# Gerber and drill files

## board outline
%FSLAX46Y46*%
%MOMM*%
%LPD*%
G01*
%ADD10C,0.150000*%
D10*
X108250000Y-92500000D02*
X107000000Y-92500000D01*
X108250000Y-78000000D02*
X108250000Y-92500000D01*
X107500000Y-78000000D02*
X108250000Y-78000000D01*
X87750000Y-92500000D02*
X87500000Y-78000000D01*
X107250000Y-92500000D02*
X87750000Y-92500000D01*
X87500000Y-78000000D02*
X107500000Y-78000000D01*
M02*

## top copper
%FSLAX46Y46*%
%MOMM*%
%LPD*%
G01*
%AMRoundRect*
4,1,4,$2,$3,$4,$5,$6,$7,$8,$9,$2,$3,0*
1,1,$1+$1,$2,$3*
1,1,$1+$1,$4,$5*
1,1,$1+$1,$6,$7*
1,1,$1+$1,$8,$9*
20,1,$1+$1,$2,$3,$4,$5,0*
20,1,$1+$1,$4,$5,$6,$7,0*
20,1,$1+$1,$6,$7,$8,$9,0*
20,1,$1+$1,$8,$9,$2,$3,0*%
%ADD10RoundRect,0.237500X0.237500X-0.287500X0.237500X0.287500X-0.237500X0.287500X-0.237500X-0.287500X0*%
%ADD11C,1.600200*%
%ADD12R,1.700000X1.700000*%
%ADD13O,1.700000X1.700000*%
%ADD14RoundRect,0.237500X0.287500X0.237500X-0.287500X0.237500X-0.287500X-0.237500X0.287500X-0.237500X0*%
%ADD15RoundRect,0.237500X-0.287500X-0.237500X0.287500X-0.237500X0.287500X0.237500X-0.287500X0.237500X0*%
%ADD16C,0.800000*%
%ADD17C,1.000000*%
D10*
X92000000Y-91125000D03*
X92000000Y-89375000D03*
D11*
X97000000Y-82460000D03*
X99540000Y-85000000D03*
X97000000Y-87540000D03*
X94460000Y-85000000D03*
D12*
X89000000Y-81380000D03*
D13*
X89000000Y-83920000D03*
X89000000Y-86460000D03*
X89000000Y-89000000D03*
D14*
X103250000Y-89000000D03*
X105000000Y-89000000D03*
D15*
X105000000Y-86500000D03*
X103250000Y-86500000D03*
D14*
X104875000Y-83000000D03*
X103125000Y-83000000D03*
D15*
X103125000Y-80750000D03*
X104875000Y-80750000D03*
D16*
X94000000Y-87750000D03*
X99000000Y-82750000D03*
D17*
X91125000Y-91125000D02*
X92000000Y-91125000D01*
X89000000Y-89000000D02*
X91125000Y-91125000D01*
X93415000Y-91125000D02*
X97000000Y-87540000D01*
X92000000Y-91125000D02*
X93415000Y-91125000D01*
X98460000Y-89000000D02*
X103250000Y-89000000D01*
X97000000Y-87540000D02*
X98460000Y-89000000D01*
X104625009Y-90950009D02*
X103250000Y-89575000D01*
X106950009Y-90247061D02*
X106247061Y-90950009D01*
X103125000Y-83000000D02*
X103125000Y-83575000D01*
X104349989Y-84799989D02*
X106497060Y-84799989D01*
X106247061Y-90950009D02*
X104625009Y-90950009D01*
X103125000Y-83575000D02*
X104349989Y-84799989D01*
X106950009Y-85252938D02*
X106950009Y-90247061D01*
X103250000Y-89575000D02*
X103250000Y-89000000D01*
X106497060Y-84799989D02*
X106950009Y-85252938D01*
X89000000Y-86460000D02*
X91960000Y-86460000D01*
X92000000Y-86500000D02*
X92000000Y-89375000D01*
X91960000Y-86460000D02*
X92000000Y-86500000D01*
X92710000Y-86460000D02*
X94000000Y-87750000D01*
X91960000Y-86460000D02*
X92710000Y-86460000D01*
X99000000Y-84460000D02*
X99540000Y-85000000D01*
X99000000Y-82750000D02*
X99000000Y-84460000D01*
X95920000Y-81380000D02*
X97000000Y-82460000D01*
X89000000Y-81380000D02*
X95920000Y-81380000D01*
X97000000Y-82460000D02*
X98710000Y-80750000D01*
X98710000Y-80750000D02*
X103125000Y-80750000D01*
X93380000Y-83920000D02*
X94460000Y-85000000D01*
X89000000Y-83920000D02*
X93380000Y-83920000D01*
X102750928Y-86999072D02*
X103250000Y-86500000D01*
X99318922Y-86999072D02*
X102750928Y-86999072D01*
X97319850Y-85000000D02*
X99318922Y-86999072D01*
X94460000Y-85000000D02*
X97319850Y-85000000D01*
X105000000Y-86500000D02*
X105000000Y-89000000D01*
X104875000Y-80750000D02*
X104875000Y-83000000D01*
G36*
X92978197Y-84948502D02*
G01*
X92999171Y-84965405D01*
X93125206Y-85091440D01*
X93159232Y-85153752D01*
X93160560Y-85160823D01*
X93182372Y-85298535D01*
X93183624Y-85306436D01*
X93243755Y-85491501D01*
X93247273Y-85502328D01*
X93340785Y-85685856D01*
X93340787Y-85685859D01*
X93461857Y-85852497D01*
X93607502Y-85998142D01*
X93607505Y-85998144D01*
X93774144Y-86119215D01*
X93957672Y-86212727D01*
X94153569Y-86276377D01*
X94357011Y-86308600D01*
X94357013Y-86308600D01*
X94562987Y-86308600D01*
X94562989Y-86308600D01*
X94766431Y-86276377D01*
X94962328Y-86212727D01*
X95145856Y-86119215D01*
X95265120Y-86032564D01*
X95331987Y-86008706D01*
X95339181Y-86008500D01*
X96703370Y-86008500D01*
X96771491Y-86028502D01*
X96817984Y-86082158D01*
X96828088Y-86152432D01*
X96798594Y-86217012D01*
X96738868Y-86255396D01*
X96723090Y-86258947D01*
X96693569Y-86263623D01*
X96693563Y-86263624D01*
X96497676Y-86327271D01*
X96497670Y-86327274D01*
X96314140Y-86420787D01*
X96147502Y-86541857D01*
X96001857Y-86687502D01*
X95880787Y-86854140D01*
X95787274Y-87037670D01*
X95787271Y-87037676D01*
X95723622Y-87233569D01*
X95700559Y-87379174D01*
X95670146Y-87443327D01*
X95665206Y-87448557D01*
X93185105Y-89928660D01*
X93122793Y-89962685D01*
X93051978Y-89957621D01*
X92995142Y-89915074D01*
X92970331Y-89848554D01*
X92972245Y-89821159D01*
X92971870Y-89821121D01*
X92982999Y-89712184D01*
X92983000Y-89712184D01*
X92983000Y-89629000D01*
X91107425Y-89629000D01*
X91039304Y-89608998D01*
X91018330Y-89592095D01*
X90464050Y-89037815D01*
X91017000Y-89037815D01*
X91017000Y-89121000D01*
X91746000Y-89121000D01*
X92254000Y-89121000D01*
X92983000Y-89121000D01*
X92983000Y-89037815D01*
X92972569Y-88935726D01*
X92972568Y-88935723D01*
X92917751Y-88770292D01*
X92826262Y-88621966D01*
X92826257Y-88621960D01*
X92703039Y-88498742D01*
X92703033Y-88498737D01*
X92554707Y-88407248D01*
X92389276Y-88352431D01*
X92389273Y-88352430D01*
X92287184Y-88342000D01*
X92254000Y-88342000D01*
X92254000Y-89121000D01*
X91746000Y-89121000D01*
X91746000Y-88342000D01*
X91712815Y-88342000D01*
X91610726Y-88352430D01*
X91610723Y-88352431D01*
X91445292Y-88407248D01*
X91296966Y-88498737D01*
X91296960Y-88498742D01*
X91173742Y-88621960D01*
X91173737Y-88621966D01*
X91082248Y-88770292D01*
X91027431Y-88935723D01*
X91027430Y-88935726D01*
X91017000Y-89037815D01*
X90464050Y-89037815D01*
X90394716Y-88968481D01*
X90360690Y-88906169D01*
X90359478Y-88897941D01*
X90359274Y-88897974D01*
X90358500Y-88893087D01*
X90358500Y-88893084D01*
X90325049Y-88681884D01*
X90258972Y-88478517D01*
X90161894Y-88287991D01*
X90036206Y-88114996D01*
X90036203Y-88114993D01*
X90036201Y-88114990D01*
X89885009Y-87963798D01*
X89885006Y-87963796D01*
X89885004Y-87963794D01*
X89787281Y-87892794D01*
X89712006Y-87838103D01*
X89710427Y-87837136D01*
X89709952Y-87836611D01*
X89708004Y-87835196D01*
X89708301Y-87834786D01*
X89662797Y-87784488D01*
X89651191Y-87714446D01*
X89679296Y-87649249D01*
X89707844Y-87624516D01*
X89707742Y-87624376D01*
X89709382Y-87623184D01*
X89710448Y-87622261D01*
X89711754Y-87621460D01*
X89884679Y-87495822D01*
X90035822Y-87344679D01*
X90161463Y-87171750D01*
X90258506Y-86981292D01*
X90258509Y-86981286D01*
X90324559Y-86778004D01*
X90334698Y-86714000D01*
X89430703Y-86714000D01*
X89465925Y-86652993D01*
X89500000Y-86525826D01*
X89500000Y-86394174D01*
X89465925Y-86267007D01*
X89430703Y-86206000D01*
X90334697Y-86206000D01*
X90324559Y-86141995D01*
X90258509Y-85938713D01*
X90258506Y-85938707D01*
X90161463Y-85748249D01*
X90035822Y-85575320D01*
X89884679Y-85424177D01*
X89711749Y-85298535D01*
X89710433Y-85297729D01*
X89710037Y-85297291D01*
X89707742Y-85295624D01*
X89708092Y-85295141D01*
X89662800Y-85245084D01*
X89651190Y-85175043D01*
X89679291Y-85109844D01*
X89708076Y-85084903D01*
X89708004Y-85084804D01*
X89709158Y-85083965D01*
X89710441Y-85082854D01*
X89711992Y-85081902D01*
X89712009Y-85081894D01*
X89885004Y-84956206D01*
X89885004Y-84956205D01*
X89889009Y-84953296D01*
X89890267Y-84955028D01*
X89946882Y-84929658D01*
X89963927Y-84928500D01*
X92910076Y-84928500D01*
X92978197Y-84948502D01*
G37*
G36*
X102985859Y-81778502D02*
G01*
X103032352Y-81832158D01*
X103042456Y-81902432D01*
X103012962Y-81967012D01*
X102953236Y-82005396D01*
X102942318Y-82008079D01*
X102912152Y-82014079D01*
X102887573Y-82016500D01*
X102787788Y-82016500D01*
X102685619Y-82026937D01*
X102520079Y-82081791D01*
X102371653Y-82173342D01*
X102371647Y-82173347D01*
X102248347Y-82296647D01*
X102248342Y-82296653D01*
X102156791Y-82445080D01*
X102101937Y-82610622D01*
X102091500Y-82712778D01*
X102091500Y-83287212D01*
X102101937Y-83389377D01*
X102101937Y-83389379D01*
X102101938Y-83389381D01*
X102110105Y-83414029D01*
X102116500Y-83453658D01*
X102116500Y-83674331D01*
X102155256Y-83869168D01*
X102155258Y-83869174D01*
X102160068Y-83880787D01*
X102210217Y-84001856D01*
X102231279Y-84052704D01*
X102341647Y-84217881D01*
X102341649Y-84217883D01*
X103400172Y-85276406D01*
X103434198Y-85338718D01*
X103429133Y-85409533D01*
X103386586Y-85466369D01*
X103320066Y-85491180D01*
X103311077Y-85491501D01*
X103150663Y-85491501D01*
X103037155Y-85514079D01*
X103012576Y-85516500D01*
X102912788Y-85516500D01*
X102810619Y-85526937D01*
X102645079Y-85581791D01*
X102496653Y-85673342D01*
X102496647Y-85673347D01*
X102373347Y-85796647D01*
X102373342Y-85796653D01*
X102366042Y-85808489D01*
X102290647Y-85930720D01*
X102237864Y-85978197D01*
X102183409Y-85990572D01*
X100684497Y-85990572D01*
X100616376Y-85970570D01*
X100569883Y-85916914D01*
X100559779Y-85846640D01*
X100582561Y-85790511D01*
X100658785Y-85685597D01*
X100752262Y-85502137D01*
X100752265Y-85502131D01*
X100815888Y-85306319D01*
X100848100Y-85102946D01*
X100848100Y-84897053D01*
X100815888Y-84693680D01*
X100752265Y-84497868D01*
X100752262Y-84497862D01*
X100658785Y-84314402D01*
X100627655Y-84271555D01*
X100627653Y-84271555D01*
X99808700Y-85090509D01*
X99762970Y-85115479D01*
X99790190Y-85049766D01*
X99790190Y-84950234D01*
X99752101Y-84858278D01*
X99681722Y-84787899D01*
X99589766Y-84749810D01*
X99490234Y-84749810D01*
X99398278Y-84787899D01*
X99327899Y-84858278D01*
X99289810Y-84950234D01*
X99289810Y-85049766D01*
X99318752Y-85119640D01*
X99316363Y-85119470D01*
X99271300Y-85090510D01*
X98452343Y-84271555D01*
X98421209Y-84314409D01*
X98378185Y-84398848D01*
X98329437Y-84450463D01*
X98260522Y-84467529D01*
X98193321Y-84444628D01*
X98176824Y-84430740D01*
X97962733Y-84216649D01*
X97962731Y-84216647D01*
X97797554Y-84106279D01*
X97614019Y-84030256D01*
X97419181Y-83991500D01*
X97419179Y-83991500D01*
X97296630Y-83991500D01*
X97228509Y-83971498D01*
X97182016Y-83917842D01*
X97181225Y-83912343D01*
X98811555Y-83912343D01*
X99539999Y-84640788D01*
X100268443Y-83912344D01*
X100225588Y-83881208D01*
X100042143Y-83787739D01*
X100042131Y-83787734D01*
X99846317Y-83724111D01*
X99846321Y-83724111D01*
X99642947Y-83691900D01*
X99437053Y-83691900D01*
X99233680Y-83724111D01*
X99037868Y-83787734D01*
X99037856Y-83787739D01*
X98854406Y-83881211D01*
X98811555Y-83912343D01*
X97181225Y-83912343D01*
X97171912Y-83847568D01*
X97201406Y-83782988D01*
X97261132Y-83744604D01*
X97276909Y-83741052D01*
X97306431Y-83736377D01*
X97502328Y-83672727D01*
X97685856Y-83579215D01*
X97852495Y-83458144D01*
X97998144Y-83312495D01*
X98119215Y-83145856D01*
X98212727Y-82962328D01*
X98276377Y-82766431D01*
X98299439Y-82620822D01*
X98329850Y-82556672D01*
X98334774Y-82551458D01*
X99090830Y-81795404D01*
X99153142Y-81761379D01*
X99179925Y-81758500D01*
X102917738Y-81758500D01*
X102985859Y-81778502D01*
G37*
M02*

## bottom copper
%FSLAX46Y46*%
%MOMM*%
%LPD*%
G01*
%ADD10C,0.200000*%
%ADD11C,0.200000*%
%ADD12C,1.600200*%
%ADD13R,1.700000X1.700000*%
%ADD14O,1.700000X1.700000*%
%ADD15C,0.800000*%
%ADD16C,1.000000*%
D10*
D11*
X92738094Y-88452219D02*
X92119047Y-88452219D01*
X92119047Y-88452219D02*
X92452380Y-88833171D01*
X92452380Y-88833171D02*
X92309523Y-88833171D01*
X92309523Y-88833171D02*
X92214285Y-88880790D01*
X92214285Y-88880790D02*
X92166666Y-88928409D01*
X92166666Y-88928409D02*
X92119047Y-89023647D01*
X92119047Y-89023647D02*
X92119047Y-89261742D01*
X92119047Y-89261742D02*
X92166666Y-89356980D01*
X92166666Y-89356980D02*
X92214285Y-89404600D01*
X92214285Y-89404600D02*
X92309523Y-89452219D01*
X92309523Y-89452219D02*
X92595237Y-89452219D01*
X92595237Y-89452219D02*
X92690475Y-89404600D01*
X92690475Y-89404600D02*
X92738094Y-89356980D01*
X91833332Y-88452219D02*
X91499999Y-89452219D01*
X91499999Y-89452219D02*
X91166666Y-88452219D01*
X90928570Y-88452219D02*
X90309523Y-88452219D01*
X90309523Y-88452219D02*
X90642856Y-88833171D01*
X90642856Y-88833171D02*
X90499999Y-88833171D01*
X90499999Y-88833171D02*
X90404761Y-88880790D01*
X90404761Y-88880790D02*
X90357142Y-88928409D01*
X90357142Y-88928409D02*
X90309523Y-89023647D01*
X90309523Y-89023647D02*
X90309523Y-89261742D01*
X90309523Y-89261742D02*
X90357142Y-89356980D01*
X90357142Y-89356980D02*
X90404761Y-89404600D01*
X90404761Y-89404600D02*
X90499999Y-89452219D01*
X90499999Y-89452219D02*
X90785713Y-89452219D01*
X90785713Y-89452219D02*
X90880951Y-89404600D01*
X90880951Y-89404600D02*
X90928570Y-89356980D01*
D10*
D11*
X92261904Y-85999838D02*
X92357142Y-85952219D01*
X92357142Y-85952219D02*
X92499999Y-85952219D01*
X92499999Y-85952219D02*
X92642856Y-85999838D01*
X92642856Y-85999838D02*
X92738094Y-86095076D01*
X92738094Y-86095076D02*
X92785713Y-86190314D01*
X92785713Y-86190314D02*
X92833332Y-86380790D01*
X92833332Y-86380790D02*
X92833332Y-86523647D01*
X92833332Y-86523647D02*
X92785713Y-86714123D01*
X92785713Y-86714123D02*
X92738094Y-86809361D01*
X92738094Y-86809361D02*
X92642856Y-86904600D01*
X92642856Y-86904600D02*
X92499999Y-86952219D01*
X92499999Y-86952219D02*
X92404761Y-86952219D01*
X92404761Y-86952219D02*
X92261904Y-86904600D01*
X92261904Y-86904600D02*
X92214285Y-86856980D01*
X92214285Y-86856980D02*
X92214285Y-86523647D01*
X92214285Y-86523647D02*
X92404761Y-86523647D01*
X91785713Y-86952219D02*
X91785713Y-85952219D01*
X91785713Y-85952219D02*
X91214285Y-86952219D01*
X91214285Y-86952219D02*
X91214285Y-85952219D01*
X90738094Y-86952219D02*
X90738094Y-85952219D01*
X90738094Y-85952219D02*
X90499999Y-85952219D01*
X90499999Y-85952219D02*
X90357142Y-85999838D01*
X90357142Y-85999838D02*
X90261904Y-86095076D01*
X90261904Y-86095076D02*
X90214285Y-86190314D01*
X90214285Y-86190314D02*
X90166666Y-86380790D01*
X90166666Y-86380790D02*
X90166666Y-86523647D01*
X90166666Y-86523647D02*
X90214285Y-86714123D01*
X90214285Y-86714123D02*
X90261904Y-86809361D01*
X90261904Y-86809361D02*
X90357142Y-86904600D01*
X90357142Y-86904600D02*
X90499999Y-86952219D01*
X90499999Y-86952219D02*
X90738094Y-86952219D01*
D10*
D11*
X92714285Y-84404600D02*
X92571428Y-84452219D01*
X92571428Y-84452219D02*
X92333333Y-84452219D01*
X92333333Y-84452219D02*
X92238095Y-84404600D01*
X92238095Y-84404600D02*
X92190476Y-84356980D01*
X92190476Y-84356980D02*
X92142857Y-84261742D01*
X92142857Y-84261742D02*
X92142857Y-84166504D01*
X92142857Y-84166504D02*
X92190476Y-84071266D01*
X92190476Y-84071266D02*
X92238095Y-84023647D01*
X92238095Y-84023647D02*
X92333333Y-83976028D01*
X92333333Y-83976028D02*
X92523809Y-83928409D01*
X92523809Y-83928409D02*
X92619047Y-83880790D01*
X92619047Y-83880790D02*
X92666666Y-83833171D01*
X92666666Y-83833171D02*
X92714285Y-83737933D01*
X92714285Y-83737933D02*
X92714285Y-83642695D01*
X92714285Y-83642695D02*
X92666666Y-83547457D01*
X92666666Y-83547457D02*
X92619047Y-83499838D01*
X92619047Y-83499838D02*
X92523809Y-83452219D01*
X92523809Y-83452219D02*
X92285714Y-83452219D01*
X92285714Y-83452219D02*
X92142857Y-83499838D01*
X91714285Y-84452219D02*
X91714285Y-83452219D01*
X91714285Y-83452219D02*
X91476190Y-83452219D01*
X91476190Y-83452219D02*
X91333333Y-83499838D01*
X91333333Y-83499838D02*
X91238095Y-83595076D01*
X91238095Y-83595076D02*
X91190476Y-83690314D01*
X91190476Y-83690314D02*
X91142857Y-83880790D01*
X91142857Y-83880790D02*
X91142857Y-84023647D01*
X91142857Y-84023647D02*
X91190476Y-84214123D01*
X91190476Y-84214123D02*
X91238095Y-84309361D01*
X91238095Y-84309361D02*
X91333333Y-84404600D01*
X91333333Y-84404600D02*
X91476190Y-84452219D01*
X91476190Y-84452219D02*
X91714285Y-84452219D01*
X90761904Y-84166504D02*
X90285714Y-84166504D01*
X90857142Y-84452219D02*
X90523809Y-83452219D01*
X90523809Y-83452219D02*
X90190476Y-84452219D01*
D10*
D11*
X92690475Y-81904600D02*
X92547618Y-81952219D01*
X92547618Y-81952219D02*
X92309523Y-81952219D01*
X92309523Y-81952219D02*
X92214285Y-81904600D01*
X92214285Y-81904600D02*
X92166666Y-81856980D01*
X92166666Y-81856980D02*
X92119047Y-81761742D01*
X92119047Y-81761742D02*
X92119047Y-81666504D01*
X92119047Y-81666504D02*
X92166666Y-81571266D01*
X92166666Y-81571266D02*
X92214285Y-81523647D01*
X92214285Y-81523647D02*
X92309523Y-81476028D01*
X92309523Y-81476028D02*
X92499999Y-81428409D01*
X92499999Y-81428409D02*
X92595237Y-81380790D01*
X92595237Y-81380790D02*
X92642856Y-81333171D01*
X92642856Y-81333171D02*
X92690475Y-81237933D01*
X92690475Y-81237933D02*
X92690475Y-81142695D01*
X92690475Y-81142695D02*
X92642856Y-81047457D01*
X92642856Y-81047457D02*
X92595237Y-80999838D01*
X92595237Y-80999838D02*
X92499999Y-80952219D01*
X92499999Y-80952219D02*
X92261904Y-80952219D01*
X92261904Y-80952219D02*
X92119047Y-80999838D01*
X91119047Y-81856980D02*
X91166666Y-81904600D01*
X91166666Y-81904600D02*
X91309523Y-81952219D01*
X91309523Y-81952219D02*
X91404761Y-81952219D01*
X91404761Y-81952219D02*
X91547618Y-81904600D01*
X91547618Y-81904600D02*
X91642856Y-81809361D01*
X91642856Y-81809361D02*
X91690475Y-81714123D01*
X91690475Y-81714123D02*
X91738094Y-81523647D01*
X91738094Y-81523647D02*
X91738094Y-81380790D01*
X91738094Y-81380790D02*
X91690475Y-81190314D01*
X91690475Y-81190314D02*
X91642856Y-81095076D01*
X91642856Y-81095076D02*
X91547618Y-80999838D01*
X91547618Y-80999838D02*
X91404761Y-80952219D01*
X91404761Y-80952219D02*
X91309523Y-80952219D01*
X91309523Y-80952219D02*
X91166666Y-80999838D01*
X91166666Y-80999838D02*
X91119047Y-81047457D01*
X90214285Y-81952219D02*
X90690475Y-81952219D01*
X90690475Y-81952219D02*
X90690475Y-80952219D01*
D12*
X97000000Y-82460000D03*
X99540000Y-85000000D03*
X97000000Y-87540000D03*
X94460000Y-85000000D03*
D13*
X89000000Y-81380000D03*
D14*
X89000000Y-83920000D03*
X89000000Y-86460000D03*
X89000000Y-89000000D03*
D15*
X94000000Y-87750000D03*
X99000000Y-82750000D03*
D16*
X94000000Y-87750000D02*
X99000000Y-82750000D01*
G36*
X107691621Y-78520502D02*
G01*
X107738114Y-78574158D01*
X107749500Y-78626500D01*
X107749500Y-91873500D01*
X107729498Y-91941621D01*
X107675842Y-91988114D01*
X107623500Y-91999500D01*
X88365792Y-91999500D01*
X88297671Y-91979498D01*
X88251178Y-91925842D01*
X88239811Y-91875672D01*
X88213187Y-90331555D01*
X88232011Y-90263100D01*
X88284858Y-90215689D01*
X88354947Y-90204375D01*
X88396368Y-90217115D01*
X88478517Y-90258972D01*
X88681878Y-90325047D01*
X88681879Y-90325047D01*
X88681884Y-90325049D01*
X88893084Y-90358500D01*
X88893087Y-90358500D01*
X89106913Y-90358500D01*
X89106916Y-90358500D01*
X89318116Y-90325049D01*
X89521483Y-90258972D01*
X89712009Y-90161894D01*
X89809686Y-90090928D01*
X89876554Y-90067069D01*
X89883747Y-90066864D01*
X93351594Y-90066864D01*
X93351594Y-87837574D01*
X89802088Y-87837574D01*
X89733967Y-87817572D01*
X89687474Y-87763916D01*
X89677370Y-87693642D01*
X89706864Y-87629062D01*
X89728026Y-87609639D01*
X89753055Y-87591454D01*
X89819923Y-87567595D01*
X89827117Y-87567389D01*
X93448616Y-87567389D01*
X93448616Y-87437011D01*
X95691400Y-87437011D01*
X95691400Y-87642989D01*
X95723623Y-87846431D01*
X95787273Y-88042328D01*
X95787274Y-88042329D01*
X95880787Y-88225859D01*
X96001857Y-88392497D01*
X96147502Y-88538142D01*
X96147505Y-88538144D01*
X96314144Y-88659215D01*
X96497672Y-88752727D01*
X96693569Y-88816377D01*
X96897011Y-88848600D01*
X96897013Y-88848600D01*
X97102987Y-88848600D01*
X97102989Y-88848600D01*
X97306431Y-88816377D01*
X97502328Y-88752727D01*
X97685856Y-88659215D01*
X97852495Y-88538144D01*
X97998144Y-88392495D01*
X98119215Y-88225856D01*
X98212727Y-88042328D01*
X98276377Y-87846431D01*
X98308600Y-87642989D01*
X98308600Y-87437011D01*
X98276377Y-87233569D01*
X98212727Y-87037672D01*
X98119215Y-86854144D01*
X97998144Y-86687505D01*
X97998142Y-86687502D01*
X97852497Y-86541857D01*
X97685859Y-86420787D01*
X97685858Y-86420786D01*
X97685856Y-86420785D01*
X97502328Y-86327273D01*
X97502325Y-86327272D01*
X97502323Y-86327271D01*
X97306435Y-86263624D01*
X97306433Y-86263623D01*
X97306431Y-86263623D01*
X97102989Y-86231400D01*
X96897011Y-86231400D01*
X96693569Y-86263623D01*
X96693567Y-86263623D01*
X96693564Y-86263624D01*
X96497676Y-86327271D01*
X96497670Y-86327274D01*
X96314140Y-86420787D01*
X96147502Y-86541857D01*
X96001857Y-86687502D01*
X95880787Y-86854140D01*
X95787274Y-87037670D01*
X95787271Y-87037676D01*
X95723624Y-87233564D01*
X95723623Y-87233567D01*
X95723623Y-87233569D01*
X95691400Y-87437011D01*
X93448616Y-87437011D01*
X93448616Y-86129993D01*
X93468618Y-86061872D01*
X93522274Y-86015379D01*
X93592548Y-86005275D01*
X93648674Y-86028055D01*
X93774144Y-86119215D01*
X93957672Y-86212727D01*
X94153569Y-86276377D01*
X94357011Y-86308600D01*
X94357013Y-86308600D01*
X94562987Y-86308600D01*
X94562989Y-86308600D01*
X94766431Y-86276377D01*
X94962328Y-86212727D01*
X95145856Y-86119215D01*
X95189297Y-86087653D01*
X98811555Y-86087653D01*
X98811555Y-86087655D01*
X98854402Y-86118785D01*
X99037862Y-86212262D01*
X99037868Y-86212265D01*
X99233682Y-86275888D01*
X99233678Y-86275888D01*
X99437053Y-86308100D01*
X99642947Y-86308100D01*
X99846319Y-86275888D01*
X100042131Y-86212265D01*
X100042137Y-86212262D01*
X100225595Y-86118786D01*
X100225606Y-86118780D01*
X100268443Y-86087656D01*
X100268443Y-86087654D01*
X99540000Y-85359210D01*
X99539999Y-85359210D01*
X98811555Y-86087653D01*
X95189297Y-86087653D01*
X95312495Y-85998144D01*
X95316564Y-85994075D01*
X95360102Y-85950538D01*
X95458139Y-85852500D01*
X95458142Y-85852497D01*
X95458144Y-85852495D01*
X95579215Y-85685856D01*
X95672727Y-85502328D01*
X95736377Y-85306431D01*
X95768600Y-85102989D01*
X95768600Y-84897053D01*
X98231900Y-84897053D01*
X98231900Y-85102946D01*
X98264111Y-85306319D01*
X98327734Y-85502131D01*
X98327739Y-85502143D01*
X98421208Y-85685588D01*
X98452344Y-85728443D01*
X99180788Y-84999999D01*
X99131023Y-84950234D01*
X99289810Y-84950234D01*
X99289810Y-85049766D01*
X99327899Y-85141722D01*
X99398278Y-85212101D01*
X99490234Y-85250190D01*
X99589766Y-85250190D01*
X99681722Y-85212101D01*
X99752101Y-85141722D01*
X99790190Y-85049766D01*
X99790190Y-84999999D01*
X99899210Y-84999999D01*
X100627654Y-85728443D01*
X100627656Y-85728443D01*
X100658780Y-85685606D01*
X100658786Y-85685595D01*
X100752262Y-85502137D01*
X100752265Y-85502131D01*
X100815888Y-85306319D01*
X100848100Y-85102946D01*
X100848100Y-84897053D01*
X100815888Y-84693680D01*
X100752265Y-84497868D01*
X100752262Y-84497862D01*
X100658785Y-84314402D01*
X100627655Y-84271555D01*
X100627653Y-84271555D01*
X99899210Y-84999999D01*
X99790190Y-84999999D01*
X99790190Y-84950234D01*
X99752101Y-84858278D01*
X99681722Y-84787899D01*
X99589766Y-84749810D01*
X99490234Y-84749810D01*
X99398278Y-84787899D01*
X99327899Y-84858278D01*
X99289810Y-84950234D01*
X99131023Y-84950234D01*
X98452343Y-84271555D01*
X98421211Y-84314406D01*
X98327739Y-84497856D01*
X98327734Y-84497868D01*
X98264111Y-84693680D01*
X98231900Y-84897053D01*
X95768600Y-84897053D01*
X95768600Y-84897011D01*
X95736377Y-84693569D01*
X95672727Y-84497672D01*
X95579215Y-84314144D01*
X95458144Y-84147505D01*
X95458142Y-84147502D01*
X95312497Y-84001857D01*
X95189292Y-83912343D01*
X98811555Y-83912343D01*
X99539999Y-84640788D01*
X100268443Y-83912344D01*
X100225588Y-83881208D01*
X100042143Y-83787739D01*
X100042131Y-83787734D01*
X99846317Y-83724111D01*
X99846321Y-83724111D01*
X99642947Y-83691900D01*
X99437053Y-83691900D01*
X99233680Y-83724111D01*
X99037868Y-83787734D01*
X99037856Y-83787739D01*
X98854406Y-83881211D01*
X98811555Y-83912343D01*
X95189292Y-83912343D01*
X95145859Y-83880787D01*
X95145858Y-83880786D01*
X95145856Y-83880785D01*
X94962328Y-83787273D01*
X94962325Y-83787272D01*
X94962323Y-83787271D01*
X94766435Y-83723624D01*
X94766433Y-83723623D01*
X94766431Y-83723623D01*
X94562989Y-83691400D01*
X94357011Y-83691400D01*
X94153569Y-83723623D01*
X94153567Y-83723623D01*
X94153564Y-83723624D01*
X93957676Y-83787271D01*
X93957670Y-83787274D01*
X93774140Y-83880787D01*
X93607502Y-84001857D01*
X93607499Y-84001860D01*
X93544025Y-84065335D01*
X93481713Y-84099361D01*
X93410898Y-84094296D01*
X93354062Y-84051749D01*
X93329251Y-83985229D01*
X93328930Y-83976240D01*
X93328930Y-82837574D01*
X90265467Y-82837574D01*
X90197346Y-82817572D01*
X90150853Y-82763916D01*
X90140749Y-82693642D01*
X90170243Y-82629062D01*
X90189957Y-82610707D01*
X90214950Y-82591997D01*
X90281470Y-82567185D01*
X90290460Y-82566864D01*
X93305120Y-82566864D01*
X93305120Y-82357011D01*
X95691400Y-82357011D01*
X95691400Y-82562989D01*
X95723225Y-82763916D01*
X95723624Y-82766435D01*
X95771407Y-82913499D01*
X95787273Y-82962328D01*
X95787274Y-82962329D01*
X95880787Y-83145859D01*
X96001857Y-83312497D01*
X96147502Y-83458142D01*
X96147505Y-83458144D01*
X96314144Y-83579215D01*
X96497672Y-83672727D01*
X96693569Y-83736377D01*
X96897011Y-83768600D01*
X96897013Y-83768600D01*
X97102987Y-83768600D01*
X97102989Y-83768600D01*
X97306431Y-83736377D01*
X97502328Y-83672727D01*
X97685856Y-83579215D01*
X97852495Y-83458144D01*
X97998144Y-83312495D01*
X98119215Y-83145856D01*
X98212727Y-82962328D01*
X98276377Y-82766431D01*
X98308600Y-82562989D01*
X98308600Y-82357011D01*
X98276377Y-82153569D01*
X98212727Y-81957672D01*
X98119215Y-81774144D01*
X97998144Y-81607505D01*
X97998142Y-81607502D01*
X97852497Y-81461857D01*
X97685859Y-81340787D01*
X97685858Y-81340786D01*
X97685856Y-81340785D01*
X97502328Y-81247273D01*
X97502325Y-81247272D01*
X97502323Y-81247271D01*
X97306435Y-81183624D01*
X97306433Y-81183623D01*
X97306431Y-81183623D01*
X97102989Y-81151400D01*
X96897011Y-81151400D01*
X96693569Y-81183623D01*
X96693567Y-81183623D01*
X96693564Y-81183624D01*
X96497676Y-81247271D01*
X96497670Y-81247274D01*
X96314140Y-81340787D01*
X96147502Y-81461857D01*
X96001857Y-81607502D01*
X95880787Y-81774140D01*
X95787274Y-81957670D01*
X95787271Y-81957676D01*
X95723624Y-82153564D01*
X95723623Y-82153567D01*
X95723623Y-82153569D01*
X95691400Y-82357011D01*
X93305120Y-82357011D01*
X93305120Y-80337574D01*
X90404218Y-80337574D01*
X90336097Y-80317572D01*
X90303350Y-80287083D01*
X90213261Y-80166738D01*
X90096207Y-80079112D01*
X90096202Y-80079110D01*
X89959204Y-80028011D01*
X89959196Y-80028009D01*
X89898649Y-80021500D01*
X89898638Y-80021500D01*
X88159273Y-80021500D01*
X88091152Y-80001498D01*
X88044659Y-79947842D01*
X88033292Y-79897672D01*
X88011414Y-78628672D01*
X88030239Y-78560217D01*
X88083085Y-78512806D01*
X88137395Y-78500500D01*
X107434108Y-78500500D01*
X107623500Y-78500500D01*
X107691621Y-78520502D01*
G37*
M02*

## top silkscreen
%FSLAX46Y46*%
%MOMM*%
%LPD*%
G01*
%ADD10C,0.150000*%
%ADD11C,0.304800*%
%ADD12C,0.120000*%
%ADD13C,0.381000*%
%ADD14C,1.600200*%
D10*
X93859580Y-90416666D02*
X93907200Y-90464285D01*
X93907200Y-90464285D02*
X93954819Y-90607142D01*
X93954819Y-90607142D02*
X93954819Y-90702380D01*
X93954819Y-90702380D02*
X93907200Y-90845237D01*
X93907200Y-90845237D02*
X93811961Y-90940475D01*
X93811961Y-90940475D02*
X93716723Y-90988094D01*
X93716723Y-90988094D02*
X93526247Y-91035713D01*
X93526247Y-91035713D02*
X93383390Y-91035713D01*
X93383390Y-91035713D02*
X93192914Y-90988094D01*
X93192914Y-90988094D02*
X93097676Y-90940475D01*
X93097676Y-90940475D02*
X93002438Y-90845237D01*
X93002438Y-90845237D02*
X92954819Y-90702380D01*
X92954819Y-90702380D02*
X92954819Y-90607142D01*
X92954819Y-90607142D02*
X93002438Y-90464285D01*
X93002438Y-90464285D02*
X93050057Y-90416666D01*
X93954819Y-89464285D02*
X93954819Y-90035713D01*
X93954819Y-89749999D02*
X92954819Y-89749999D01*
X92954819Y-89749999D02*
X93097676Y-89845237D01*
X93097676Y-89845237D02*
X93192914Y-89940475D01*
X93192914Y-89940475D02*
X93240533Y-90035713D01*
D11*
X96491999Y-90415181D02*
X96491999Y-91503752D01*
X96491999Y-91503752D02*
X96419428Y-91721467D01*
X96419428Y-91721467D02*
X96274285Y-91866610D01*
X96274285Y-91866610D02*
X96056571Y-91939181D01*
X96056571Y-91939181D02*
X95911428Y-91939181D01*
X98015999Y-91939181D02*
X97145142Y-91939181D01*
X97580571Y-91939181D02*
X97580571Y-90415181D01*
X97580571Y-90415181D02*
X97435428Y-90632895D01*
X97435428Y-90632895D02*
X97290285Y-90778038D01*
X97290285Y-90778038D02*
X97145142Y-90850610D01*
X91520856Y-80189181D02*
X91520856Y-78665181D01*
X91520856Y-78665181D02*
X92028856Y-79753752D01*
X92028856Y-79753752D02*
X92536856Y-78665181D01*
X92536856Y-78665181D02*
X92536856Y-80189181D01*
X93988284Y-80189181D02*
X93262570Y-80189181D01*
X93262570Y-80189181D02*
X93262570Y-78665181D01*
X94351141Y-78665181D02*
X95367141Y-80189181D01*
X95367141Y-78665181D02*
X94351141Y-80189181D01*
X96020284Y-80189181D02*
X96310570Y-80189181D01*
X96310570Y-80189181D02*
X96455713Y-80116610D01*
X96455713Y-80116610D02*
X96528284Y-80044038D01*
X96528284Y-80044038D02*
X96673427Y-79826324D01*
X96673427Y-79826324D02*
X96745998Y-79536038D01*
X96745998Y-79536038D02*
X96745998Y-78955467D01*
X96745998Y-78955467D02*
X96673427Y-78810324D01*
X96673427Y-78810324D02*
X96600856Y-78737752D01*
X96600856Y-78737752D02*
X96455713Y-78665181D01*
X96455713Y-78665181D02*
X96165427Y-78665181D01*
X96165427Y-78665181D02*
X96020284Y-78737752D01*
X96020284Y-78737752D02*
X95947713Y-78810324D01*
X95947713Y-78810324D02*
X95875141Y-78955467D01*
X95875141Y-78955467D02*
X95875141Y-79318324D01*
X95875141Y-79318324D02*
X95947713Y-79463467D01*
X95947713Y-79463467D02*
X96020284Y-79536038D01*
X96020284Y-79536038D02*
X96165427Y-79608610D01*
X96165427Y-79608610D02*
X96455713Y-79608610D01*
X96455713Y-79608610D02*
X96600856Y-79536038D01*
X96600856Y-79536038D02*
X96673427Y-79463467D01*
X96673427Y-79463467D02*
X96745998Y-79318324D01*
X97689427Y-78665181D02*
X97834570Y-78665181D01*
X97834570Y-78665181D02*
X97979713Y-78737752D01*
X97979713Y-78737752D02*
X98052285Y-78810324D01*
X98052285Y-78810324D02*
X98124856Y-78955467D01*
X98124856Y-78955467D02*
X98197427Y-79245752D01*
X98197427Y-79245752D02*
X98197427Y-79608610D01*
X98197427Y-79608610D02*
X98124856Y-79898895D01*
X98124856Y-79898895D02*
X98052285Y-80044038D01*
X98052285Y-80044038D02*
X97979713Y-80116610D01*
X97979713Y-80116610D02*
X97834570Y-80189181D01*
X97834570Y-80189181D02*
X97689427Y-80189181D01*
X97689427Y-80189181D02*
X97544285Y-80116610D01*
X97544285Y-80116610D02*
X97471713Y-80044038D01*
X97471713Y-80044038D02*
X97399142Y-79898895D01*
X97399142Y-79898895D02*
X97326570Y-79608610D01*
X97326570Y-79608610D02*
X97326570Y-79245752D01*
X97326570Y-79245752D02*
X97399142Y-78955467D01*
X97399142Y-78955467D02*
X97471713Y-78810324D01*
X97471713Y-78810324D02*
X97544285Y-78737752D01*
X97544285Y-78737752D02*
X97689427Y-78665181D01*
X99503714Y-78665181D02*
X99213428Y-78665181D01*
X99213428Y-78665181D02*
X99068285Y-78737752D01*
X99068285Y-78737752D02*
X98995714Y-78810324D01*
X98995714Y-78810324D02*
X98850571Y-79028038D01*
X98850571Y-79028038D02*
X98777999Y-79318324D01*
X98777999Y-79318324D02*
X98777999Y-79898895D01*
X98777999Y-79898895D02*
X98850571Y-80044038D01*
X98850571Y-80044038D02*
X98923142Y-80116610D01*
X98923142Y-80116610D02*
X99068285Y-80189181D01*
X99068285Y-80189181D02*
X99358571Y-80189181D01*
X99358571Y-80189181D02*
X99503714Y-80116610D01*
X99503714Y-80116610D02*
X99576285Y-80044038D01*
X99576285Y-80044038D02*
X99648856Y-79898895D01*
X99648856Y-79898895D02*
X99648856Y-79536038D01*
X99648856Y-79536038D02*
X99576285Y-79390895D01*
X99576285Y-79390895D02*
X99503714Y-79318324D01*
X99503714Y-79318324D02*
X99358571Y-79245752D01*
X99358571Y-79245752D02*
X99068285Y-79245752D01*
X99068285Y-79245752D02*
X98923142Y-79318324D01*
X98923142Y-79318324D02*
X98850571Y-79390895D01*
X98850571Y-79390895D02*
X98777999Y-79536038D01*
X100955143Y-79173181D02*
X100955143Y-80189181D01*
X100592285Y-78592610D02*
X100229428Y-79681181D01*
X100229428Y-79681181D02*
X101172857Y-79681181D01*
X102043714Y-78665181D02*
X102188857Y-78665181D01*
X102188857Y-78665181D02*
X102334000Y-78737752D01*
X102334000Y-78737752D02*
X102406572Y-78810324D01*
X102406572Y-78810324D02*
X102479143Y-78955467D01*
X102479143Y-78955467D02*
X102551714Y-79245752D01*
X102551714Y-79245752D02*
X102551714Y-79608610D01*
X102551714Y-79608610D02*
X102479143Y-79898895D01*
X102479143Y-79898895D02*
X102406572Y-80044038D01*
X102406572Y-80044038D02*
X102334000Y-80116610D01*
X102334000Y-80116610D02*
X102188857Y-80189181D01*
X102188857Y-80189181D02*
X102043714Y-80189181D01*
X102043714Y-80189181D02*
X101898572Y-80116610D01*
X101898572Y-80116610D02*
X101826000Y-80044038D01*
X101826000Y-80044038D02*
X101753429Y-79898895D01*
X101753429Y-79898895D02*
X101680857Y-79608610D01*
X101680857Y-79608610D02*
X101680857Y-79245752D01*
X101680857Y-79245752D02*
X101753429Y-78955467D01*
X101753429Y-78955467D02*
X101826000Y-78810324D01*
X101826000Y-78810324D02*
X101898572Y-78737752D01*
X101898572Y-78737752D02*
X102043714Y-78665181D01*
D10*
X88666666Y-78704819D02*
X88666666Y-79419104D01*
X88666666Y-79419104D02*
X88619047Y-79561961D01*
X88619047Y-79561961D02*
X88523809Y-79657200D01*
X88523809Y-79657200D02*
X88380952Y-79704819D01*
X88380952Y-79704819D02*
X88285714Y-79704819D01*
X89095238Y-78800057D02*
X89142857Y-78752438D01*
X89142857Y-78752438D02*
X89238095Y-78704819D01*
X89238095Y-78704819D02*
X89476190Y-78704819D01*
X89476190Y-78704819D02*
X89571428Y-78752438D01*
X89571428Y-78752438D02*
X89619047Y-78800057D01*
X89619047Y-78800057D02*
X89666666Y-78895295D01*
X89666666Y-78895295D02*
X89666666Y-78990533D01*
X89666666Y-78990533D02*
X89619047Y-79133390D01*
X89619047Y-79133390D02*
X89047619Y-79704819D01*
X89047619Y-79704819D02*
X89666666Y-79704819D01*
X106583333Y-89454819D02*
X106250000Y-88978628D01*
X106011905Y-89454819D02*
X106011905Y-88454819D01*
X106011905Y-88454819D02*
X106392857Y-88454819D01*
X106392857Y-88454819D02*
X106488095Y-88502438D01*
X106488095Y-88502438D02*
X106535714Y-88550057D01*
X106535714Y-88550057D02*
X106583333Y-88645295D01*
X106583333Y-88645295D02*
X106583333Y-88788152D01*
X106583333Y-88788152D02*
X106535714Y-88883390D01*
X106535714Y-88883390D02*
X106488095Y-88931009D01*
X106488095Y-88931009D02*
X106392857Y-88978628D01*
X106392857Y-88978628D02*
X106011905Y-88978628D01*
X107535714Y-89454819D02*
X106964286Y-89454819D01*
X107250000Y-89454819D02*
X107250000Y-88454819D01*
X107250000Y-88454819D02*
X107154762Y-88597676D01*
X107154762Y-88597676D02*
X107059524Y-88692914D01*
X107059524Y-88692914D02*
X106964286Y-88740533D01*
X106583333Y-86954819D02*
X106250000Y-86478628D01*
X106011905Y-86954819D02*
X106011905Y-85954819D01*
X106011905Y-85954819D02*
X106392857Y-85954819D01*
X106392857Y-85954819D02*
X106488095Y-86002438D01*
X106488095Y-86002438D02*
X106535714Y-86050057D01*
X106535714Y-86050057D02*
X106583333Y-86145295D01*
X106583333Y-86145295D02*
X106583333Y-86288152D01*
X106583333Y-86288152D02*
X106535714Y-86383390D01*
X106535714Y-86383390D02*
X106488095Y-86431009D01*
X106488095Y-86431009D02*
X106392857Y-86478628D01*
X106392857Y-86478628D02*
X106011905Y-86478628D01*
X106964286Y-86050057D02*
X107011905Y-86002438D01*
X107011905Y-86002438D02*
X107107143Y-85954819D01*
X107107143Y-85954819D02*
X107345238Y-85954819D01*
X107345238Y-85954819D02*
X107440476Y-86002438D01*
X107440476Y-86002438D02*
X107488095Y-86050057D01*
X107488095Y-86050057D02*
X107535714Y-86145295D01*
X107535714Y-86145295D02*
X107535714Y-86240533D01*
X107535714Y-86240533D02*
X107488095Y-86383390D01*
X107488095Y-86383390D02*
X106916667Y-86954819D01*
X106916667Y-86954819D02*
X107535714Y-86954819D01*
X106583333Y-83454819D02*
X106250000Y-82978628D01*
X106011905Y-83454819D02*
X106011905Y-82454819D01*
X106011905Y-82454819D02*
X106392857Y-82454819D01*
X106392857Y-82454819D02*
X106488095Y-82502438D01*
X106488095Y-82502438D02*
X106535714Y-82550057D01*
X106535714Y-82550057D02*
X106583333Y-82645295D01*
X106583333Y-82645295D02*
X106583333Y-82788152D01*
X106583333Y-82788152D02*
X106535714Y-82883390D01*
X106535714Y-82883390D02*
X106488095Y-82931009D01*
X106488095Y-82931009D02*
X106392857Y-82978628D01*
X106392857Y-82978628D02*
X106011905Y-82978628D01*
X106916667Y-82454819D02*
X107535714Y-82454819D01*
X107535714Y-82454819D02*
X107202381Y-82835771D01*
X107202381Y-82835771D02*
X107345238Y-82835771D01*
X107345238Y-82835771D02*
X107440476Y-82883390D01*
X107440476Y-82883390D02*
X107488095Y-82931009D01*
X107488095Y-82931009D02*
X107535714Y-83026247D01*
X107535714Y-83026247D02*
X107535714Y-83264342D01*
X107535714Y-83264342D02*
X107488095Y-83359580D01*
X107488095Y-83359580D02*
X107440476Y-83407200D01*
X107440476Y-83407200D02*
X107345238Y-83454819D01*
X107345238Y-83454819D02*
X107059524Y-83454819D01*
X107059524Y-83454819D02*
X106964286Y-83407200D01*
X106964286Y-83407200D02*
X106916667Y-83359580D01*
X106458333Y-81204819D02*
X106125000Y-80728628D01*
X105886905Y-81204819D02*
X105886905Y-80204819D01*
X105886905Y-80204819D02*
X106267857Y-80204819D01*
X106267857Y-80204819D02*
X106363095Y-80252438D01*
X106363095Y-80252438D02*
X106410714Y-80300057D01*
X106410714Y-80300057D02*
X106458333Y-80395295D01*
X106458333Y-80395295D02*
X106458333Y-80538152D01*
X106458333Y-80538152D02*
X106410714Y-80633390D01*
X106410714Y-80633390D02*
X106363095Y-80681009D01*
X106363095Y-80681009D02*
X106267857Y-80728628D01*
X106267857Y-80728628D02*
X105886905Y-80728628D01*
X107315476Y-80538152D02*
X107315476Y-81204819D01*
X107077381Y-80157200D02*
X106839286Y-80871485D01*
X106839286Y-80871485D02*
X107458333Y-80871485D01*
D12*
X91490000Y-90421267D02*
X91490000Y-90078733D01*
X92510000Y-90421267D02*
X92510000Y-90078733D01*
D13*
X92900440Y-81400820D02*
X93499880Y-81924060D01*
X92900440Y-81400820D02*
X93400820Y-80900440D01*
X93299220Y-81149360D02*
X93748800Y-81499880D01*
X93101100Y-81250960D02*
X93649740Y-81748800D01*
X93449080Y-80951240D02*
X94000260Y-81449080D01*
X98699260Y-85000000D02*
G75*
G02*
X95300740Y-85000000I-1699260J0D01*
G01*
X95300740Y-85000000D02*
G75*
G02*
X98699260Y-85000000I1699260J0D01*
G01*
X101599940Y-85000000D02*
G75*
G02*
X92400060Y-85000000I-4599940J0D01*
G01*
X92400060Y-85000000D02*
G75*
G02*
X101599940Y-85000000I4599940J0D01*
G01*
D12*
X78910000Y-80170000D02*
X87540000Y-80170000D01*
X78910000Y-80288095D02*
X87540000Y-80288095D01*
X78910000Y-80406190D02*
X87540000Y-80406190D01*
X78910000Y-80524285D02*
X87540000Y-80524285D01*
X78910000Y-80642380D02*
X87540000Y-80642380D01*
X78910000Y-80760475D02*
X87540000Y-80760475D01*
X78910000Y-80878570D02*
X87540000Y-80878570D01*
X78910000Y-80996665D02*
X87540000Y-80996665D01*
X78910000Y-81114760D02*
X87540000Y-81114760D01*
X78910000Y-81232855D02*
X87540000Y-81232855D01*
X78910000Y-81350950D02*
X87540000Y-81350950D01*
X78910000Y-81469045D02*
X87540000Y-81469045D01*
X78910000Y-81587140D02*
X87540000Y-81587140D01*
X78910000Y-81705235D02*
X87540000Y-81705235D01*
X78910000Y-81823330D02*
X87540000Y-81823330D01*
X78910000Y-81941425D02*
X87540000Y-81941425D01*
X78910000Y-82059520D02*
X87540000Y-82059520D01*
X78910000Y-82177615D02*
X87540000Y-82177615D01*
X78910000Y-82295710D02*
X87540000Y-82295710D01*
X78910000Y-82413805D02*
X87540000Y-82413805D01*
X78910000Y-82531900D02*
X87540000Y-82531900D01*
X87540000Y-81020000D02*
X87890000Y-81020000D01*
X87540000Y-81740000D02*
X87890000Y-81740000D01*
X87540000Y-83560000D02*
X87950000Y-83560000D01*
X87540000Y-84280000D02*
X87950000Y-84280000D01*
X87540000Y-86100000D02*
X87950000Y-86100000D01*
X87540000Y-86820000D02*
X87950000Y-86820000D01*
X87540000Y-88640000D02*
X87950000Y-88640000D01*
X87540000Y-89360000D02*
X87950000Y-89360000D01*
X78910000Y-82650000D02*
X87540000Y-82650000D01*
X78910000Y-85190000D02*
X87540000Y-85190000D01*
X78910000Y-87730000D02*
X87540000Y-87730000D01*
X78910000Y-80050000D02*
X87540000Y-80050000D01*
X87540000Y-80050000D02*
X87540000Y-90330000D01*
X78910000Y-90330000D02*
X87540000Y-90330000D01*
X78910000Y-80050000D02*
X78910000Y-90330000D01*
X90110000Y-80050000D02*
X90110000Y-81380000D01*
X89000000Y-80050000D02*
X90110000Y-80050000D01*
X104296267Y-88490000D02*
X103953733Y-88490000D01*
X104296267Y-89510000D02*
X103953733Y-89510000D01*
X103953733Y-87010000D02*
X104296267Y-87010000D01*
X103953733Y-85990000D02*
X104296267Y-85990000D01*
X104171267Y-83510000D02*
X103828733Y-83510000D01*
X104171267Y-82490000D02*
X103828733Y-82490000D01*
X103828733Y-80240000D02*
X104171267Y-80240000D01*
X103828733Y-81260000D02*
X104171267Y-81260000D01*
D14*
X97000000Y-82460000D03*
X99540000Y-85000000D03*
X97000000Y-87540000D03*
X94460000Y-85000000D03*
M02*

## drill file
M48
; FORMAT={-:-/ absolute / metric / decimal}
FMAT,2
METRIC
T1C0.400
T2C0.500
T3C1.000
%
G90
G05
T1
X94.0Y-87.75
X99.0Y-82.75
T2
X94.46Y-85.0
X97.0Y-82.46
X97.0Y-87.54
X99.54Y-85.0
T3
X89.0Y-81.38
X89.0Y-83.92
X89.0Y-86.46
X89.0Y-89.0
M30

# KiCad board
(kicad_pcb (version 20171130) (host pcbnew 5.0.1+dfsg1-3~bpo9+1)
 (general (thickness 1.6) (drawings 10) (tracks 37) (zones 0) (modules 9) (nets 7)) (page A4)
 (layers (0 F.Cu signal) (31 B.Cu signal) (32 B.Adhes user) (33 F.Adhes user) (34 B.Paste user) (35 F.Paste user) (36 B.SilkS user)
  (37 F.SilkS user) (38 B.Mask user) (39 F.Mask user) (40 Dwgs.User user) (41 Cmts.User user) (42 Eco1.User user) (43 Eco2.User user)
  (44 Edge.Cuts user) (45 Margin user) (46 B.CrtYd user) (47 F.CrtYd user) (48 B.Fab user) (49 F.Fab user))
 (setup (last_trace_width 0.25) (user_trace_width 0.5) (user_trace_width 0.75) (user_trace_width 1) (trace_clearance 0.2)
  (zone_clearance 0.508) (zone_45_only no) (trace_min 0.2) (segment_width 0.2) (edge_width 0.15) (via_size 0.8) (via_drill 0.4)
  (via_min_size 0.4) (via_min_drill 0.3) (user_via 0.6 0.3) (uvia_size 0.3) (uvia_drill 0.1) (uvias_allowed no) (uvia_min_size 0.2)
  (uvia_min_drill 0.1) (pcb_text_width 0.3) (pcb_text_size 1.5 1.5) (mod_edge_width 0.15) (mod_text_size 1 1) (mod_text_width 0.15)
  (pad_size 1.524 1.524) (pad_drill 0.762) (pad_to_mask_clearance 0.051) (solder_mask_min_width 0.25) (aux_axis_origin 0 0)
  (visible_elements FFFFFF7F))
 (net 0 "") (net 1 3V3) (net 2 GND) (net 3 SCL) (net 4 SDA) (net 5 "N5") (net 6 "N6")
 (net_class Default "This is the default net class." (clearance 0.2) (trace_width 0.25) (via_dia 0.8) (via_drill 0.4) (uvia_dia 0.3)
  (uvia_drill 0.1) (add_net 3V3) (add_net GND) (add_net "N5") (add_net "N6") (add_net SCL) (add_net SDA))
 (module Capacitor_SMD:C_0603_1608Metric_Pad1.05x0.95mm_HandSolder (layer F.Cu) (at 92 90.25 90)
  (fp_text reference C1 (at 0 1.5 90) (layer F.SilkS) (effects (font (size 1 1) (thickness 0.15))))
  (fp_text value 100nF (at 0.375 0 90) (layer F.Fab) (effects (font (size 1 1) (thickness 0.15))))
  (fp_line (start -0.171267 -0.51) (end 0.171267 -0.51) (layer F.SilkS) (width 0.12))
  (fp_line (start -0.171267 0.51) (end 0.171267 0.51) (layer F.SilkS) (width 0.12))
  (pad 1 smd roundrect (at -0.875 0 90) (size 1.05 0.95) (layers F.Cu F.Paste F.Mask) (roundrect_rratio 0.25) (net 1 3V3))
  (pad 2 smd roundrect (at 0.875 0 90) (size 1.05 0.95) (layers F.Cu F.Paste F.Mask) (roundrect_rratio 0.25) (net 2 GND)))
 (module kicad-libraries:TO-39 (layer F.Cu) (at 97 85)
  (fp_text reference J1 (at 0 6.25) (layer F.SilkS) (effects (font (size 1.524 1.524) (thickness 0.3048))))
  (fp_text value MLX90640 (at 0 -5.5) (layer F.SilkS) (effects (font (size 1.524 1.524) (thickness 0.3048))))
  (fp_line (start -4.09956 -3.59918) (end -3.50012 -3.07594) (layer F.SilkS) (width 0.381))
  (fp_line (start -4.09956 -3.59918) (end -3.59918 -4.09956) (layer F.SilkS) (width 0.381))
  (fp_line (start -3.70078 -3.85064) (end -3.2512 -3.50012) (layer F.SilkS) (width 0.381))
  (fp_line (start -3.8989 -3.74904) (end -3.35026 -3.2512) (layer F.SilkS) (width 0.381))
  (fp_line (start -3.55092 -4.04876) (end -2.99974 -3.55092) (layer F.SilkS) (width 0.381))
  (fp_circle (center 0 0) (end 1.69926 0) (layer F.SilkS) (width 0.381))
  (fp_circle (center 0 0) (end 4.59994 0) (layer F.SilkS) (width 0.381))
  (pad 4 thru_hole circle (at 0 -2.54) (size 1.6002 1.6002) (drill 0.50038) (layers *.Cu *.Mask F.SilkS) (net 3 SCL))
  (pad 3 thru_hole circle (at 2.54 0) (size 1.6002 1.6002) (drill 0.50038) (layers *.Cu *.Mask F.SilkS) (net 2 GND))
  (pad 2 thru_hole circle (at 0 2.54) (size 1.6002 1.6002) (drill 0.50038) (layers *.Cu *.Mask F.SilkS) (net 1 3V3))
  (pad 1 thru_hole circle (at -2.54 0) (size 1.6002 1.6002) (drill 0.50038) (layers *.Cu *.Mask F.SilkS) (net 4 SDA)))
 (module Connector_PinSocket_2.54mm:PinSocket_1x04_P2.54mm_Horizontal (layer F.Cu) (at 89 81.38)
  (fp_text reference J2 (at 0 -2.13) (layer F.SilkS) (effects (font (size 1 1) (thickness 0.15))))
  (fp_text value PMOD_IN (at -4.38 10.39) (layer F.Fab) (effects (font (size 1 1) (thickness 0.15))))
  (fp_line (start -10.09 -1.21) (end -1.46 -1.21) (layer F.SilkS) (width 0.12))
  (fp_line (start -10.09 -1.091905) (end -1.46 -1.091905) (layer F.SilkS) (width 0.12))
  (fp_line (start -10.09 -0.97381) (end -1.46 -0.97381) (layer F.SilkS) (width 0.12))
  (fp_line (start -10.09 -0.855715) (end -1.46 -0.855715) (layer F.SilkS) (width 0.12))
  (fp_line (start -10.09 -0.73762) (end -1.46 -0.73762) (layer F.SilkS) (width 0.12))
  (fp_line (start -10.09 -0.619525) (end -1.46 -0.619525) (layer F.SilkS) (width 0.12))
  (fp_line (start -10.09 -0.50143) (end -1.46 -0.50143) (layer F.SilkS) (width 0.12))
  (fp_line (start -10.09 -0.383335) (end -1.46 -0.383335) (layer F.SilkS) (width 0.12))
  (fp_line (start -10.09 -0.26524) (end -1.46 -0.26524) (layer F.SilkS) (width 0.12))
  (fp_line (start -10.09 -0.147145) (end -1.46 -0.147145) (layer F.SilkS) (width 0.12))
  (fp_line (start -10.09 -0.02905) (end -1.46 -0.02905) (layer F.SilkS) (width 0.12))
  (fp_line (start -10.09 0.089045) (end -1.46 0.089045) (layer F.SilkS) (width 0.12))
  (fp_line (start -10.09 0.20714) (end -1.46 0.20714) (layer F.SilkS) (width 0.12))
  (fp_line (start -10.09 0.325235) (end -1.46 0.325235) (layer F.SilkS) (width 0.12))
  (fp_line (start -10.09 0.44333) (end -1.46 0.44333) (layer F.SilkS) (width 0.12))
  (fp_line (start -10.09 0.561425) (end -1.46 0.561425) (layer F.SilkS) (width 0.12))
  (fp_line (start -10.09 0.67952) (end -1.46 0.67952) (layer F.SilkS) (width 0.12))
  (fp_line (start -10.09 0.797615) (end -1.46 0.797615) (layer F.SilkS) (width 0.12))
  (fp_line (start -10.09 0.91571) (end -1.46 0.91571) (layer F.SilkS) (width 0.12))
  (fp_line (start -10.09 1.033805) (end -1.46 1.033805) (layer F.SilkS) (width 0.12))
  (fp_line (start -10.09 1.1519) (end -1.46 1.1519) (layer F.SilkS) (width 0.12))
  (fp_line (start -1.46 -0.36) (end -1.11 -0.36) (layer F.SilkS) (width 0.12))
  (fp_line (start -1.46 0.36) (end -1.11 0.36) (layer F.SilkS) (width 0.12))
  (fp_line (start -1.46 2.18) (end -1.05 2.18) (layer F.SilkS) (width 0.12))
  (fp_line (start -1.46 2.9) (end -1.05 2.9) (layer F.SilkS) (width 0.12))
  (fp_line (start -1.46 4.72) (end -1.05 4.72) (layer F.SilkS) (width 0.12))
  (fp_line (start -1.46 5.44) (end -1.05 5.44) (layer F.SilkS) (width 0.12))
  (fp_line (start -1.46 7.26) (end -1.05 7.26) (layer F.SilkS) (width 0.12))
  (fp_line (start -1.46 7.98) (end -1.05 7.98) (layer F.SilkS) (width 0.12))
  (fp_line (start -10.09 1.27) (end -1.46 1.27) (layer F.SilkS) (width 0.12))
  (fp_line (start -10.09 3.81) (end -1.46 3.81) (layer F.SilkS) (width 0.12))
  (fp_line (start -10.09 6.35) (end -1.46 6.35) (layer F.SilkS) (width 0.12))
  (fp_line (start -10.09 -1.33) (end -1.46 -1.33) (layer F.SilkS) (width 0.12))
  (fp_line (start -1.46 -1.33) (end -1.46 8.95) (layer F.SilkS) (width 0.12))
  (fp_line (start -10.09 8.95) (end -1.46 8.95) (layer F.SilkS) (width 0.12))
  (fp_line (start -10.09 -1.33) (end -10.09 8.95) (layer F.SilkS) (width 0.12))
  (fp_line (start 1.11 -1.33) (end 1.11 0) (layer F.SilkS) (width 0.12))
  (fp_line (start 0 -1.33) (end 1.11 -1.33) (layer F.SilkS) (width 0.12))
  (pad 1 thru_hole rect (at 0 0) (size 1.7 1.7) (drill 1) (layers *.Cu *.Mask) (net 3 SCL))
  (pad 2 thru_hole oval (at 0 2.54) (size 1.7 1.7) (drill 1) (layers *.Cu *.Mask) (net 4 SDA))
  (pad 3 thru_hole oval (at 0 5.08) (size 1.7 1.7) (drill 1) (layers *.Cu *.Mask) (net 2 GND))
  (pad 4 thru_hole oval (at 0 7.62) (size 1.7 1.7) (drill 1) (layers *.Cu *.Mask) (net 1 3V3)))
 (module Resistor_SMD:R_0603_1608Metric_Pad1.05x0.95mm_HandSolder (layer F.Cu) (at 104.125 89 180)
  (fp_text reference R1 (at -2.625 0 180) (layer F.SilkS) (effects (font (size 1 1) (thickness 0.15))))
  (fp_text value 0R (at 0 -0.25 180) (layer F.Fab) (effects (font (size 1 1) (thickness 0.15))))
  (fp_line (start -0.171267 0.51) (end 0.171267 0.51) (layer F.SilkS) (width 0.12))
  (fp_line (start -0.171267 -0.51) (end 0.171267 -0.51) (layer F.SilkS) (width 0.12))
  (pad 2 smd roundrect (at 0.875 0 180) (size 1.05 0.95) (layers F.Cu F.Paste F.Mask) (roundrect_rratio 0.25) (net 1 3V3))
  (pad 1 smd roundrect (at -0.875 0 180) (size 1.05 0.95) (layers F.Cu F.Paste F.Mask) (roundrect_rratio 0.25) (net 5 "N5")))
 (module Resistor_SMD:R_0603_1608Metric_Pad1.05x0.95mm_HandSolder (layer F.Cu) (at 104.125 86.5)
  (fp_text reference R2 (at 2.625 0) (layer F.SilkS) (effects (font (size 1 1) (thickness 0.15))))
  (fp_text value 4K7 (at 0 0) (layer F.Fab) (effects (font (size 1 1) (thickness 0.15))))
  (fp_line (start -0.171267 0.51) (end 0.171267 0.51) (layer F.SilkS) (width 0.12))
  (fp_line (start -0.171267 -0.51) (end 0.171267 -0.51) (layer F.SilkS) (width 0.12))
  (pad 2 smd roundrect (at 0.875 0) (size 1.05 0.95) (layers F.Cu F.Paste F.Mask) (roundrect_rratio 0.25) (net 5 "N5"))
  (pad 1 smd roundrect (at -0.875 0) (size 1.05 0.95) (layers F.Cu F.Paste F.Mask) (roundrect_rratio 0.25) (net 4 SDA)))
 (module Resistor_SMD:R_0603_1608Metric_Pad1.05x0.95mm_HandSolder (layer F.Cu) (at 104 83 180)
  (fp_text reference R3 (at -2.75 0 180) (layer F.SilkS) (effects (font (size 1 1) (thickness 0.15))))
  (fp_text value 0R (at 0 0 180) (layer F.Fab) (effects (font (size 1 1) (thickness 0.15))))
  (fp_line (start -0.171267 -0.51) (end 0.171267 -0.51) (layer F.SilkS) (width 0.12))
  (fp_line (start -0.171267 0.51) (end 0.171267 0.51) (layer F.SilkS) (width 0.12))
  (pad 1 smd roundrect (at -0.875 0 180) (size 1.05 0.95) (layers F.Cu F.Paste F.Mask) (roundrect_rratio 0.25) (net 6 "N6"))
  (pad 2 smd roundrect (at 0.875 0 180) (size 1.05 0.95) (layers F.Cu F.Paste F.Mask) (roundrect_rratio 0.25) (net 1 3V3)))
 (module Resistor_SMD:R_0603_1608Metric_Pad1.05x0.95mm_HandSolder (layer F.Cu) (at 104 80.75)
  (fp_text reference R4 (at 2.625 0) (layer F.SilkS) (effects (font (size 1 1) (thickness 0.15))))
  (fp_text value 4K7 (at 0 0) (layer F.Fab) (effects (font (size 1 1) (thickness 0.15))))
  (fp_line (start -0.171267 -0.51) (end 0.171267 -0.51) (layer F.SilkS) (width 0.12))
  (fp_line (start -0.171267 0.51) (end 0.171267 0.51) (layer F.SilkS) (width 0.12))
  (pad 1 smd roundrect (at -0.875 0) (size 1.05 0.95) (layers F.Cu F.Paste F.Mask) (roundrect_rratio 0.25) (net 3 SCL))
  (pad 2 smd roundrect (at 0.875 0) (size 1.05 0.95) (layers F.Cu F.Paste F.Mask) (roundrect_rratio 0.25) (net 6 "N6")))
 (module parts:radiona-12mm (layer B.Cu) (at 102.5 80.5 180)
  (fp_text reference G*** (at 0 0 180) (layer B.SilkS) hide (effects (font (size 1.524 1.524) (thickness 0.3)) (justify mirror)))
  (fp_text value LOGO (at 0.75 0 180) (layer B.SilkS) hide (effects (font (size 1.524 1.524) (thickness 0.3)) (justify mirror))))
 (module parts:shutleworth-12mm (layer B.Cu) (at 101.75 90.25 180)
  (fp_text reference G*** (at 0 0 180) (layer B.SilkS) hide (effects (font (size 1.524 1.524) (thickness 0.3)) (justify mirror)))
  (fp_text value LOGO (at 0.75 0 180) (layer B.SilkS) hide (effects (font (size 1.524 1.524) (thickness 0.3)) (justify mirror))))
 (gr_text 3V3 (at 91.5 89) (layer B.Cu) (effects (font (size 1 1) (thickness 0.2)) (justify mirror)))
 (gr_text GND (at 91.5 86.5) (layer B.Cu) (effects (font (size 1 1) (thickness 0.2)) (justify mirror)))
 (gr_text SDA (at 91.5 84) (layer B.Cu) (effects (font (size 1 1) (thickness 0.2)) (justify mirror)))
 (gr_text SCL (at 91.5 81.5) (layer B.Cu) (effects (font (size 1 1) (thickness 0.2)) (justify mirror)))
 (gr_line (start 108.25 92.5) (end 107 92.5) (layer Edge.Cuts) (width 0.15))
 (gr_line (start 108.25 78) (end 108.25 92.5) (layer Edge.Cuts) (width 0.15))
 (gr_line (start 107.5 78) (end 108.25 78) (layer Edge.Cuts) (width 0.15))
 (gr_line (start 87.75 92.5) (end 87.5 78) (layer Edge.Cuts) (width 0.15))
 (gr_line (start 107.25 92.5) (end 87.75 92.5) (layer Edge.Cuts) (width 0.15))
 (gr_line (start 87.5 78) (end 107.5 78) (layer Edge.Cuts) (width 0.15))
 (segment (start 91.125 91.125) (end 92 91.125) (width 1) (layer F.Cu) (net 1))
 (segment (start 89 89) (end 91.125 91.125) (width 1) (layer F.Cu) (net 1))
 (segment (start 93.415 91.125) (end 97 87.54) (width 1) (layer F.Cu) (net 1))
 (segment (start 92 91.125) (end 93.415 91.125) (width 1) (layer F.Cu) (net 1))
 (segment (start 98.46 89) (end 103.25 89) (width 1) (layer F.Cu) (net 1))
 (segment (start 97 87.54) (end 98.46 89) (width 1) (layer F.Cu) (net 1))
 (segment (start 104.625009 90.950009) (end 103.25 89.575) (width 1) (layer F.Cu) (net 1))
 (segment (start 106.950009 90.247061) (end 106.247061 90.950009) (width 1) (layer F.Cu) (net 1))
 (segment (start 103.125 83) (end 103.125 83.575) (width 1) (layer F.Cu) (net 1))
 (segment (start 104.349989 84.799989) (end 106.49706 84.799989) (width 1) (layer F.Cu) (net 1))
 (segment (start 106.247061 90.950009) (end 104.625009 90.950009) (width 1) (layer F.Cu) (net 1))
 (segment (start 103.125 83.575) (end 104.349989 84.799989) (width 1) (layer F.Cu) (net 1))
 (segment (start 106.950009 85.252938) (end 106.950009 90.247061) (width 1) (layer F.Cu) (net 1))
 (segment (start 103.25 89.575) (end 103.25 89) (width 1) (layer F.Cu) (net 1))
 (segment (start 106.49706 84.799989) (end 106.950009 85.252938) (width 1) (layer F.Cu) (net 1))
 (segment (start 89 86.46) (end 91.96 86.46) (width 1) (layer F.Cu) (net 2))
 (segment (start 92 86.5) (end 92 89.375) (width 1) (layer F.Cu) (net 2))
 (segment (start 91.96 86.46) (end 92 86.5) (width 1) (layer F.Cu) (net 2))
 (via (at 94 87.75) (size 0.8) (drill 0.4) (layers F.Cu B.Cu) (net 2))
 (segment (start 92.71 86.46) (end 94 87.75) (width 1) (layer F.Cu) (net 2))
 (segment (start 91.96 86.46) (end 92.71 86.46) (width 1) (layer F.Cu) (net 2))
 (via (at 99 82.75) (size 0.8) (drill 0.4) (layers F.Cu B.Cu) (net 2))
 (segment (start 94 87.75) (end 99 82.75) (width 1) (layer B.Cu) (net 2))
 (segment (start 99 84.46) (end 99.54 85) (width 1) (layer F.Cu) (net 2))
 (segment (start 99 82.75) (end 99 84.46) (width 1) (layer F.Cu) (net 2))
 (segment (start 95.92 81.38) (end 97 82.46) (width 1) (layer F.Cu) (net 3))
 (segment (start 89 81.38) (end 95.92 81.38) (width 1) (layer F.Cu) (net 3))
 (segment (start 97 82.46) (end 98.71 80.75) (width 1) (layer F.Cu) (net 3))
 (segment (start 98.71 80.75) (end 103.125 80.75) (width 1) (layer F.Cu) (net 3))
 (segment (start 93.38 83.92) (end 94.46 85) (width 1) (layer F.Cu) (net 4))
 (segment (start 89 83.92) (end 93.38 83.92) (width 1) (layer F.Cu) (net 4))
 (segment (start 102.750928 86.999072) (end 103.25 86.5) (width 1) (layer F.Cu) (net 4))
 (segment (start 99.318922 86.999072) (end 102.750928 86.999072) (width 1) (layer F.Cu) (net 4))
 (segment (start 97.31985 85) (end 99.318922 86.999072) (width 1) (layer F.Cu) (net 4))
 (segment (start 94.46 85) (end 97.31985 85) (width 1) (layer F.Cu) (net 4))
 (segment (start 105 86.5) (end 105 89) (width 1) (layer F.Cu) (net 5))
 (segment (start 104.875 80.75) (end 104.875 83) (width 1) (layer F.Cu) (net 6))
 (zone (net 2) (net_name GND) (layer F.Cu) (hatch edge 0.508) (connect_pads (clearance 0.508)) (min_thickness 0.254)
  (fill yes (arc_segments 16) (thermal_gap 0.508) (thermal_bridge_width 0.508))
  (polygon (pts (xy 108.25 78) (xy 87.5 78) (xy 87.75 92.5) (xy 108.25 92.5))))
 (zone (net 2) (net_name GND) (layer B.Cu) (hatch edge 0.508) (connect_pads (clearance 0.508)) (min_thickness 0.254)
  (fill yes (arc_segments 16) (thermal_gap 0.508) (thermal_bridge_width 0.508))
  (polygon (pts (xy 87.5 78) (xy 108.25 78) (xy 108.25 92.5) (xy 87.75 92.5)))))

